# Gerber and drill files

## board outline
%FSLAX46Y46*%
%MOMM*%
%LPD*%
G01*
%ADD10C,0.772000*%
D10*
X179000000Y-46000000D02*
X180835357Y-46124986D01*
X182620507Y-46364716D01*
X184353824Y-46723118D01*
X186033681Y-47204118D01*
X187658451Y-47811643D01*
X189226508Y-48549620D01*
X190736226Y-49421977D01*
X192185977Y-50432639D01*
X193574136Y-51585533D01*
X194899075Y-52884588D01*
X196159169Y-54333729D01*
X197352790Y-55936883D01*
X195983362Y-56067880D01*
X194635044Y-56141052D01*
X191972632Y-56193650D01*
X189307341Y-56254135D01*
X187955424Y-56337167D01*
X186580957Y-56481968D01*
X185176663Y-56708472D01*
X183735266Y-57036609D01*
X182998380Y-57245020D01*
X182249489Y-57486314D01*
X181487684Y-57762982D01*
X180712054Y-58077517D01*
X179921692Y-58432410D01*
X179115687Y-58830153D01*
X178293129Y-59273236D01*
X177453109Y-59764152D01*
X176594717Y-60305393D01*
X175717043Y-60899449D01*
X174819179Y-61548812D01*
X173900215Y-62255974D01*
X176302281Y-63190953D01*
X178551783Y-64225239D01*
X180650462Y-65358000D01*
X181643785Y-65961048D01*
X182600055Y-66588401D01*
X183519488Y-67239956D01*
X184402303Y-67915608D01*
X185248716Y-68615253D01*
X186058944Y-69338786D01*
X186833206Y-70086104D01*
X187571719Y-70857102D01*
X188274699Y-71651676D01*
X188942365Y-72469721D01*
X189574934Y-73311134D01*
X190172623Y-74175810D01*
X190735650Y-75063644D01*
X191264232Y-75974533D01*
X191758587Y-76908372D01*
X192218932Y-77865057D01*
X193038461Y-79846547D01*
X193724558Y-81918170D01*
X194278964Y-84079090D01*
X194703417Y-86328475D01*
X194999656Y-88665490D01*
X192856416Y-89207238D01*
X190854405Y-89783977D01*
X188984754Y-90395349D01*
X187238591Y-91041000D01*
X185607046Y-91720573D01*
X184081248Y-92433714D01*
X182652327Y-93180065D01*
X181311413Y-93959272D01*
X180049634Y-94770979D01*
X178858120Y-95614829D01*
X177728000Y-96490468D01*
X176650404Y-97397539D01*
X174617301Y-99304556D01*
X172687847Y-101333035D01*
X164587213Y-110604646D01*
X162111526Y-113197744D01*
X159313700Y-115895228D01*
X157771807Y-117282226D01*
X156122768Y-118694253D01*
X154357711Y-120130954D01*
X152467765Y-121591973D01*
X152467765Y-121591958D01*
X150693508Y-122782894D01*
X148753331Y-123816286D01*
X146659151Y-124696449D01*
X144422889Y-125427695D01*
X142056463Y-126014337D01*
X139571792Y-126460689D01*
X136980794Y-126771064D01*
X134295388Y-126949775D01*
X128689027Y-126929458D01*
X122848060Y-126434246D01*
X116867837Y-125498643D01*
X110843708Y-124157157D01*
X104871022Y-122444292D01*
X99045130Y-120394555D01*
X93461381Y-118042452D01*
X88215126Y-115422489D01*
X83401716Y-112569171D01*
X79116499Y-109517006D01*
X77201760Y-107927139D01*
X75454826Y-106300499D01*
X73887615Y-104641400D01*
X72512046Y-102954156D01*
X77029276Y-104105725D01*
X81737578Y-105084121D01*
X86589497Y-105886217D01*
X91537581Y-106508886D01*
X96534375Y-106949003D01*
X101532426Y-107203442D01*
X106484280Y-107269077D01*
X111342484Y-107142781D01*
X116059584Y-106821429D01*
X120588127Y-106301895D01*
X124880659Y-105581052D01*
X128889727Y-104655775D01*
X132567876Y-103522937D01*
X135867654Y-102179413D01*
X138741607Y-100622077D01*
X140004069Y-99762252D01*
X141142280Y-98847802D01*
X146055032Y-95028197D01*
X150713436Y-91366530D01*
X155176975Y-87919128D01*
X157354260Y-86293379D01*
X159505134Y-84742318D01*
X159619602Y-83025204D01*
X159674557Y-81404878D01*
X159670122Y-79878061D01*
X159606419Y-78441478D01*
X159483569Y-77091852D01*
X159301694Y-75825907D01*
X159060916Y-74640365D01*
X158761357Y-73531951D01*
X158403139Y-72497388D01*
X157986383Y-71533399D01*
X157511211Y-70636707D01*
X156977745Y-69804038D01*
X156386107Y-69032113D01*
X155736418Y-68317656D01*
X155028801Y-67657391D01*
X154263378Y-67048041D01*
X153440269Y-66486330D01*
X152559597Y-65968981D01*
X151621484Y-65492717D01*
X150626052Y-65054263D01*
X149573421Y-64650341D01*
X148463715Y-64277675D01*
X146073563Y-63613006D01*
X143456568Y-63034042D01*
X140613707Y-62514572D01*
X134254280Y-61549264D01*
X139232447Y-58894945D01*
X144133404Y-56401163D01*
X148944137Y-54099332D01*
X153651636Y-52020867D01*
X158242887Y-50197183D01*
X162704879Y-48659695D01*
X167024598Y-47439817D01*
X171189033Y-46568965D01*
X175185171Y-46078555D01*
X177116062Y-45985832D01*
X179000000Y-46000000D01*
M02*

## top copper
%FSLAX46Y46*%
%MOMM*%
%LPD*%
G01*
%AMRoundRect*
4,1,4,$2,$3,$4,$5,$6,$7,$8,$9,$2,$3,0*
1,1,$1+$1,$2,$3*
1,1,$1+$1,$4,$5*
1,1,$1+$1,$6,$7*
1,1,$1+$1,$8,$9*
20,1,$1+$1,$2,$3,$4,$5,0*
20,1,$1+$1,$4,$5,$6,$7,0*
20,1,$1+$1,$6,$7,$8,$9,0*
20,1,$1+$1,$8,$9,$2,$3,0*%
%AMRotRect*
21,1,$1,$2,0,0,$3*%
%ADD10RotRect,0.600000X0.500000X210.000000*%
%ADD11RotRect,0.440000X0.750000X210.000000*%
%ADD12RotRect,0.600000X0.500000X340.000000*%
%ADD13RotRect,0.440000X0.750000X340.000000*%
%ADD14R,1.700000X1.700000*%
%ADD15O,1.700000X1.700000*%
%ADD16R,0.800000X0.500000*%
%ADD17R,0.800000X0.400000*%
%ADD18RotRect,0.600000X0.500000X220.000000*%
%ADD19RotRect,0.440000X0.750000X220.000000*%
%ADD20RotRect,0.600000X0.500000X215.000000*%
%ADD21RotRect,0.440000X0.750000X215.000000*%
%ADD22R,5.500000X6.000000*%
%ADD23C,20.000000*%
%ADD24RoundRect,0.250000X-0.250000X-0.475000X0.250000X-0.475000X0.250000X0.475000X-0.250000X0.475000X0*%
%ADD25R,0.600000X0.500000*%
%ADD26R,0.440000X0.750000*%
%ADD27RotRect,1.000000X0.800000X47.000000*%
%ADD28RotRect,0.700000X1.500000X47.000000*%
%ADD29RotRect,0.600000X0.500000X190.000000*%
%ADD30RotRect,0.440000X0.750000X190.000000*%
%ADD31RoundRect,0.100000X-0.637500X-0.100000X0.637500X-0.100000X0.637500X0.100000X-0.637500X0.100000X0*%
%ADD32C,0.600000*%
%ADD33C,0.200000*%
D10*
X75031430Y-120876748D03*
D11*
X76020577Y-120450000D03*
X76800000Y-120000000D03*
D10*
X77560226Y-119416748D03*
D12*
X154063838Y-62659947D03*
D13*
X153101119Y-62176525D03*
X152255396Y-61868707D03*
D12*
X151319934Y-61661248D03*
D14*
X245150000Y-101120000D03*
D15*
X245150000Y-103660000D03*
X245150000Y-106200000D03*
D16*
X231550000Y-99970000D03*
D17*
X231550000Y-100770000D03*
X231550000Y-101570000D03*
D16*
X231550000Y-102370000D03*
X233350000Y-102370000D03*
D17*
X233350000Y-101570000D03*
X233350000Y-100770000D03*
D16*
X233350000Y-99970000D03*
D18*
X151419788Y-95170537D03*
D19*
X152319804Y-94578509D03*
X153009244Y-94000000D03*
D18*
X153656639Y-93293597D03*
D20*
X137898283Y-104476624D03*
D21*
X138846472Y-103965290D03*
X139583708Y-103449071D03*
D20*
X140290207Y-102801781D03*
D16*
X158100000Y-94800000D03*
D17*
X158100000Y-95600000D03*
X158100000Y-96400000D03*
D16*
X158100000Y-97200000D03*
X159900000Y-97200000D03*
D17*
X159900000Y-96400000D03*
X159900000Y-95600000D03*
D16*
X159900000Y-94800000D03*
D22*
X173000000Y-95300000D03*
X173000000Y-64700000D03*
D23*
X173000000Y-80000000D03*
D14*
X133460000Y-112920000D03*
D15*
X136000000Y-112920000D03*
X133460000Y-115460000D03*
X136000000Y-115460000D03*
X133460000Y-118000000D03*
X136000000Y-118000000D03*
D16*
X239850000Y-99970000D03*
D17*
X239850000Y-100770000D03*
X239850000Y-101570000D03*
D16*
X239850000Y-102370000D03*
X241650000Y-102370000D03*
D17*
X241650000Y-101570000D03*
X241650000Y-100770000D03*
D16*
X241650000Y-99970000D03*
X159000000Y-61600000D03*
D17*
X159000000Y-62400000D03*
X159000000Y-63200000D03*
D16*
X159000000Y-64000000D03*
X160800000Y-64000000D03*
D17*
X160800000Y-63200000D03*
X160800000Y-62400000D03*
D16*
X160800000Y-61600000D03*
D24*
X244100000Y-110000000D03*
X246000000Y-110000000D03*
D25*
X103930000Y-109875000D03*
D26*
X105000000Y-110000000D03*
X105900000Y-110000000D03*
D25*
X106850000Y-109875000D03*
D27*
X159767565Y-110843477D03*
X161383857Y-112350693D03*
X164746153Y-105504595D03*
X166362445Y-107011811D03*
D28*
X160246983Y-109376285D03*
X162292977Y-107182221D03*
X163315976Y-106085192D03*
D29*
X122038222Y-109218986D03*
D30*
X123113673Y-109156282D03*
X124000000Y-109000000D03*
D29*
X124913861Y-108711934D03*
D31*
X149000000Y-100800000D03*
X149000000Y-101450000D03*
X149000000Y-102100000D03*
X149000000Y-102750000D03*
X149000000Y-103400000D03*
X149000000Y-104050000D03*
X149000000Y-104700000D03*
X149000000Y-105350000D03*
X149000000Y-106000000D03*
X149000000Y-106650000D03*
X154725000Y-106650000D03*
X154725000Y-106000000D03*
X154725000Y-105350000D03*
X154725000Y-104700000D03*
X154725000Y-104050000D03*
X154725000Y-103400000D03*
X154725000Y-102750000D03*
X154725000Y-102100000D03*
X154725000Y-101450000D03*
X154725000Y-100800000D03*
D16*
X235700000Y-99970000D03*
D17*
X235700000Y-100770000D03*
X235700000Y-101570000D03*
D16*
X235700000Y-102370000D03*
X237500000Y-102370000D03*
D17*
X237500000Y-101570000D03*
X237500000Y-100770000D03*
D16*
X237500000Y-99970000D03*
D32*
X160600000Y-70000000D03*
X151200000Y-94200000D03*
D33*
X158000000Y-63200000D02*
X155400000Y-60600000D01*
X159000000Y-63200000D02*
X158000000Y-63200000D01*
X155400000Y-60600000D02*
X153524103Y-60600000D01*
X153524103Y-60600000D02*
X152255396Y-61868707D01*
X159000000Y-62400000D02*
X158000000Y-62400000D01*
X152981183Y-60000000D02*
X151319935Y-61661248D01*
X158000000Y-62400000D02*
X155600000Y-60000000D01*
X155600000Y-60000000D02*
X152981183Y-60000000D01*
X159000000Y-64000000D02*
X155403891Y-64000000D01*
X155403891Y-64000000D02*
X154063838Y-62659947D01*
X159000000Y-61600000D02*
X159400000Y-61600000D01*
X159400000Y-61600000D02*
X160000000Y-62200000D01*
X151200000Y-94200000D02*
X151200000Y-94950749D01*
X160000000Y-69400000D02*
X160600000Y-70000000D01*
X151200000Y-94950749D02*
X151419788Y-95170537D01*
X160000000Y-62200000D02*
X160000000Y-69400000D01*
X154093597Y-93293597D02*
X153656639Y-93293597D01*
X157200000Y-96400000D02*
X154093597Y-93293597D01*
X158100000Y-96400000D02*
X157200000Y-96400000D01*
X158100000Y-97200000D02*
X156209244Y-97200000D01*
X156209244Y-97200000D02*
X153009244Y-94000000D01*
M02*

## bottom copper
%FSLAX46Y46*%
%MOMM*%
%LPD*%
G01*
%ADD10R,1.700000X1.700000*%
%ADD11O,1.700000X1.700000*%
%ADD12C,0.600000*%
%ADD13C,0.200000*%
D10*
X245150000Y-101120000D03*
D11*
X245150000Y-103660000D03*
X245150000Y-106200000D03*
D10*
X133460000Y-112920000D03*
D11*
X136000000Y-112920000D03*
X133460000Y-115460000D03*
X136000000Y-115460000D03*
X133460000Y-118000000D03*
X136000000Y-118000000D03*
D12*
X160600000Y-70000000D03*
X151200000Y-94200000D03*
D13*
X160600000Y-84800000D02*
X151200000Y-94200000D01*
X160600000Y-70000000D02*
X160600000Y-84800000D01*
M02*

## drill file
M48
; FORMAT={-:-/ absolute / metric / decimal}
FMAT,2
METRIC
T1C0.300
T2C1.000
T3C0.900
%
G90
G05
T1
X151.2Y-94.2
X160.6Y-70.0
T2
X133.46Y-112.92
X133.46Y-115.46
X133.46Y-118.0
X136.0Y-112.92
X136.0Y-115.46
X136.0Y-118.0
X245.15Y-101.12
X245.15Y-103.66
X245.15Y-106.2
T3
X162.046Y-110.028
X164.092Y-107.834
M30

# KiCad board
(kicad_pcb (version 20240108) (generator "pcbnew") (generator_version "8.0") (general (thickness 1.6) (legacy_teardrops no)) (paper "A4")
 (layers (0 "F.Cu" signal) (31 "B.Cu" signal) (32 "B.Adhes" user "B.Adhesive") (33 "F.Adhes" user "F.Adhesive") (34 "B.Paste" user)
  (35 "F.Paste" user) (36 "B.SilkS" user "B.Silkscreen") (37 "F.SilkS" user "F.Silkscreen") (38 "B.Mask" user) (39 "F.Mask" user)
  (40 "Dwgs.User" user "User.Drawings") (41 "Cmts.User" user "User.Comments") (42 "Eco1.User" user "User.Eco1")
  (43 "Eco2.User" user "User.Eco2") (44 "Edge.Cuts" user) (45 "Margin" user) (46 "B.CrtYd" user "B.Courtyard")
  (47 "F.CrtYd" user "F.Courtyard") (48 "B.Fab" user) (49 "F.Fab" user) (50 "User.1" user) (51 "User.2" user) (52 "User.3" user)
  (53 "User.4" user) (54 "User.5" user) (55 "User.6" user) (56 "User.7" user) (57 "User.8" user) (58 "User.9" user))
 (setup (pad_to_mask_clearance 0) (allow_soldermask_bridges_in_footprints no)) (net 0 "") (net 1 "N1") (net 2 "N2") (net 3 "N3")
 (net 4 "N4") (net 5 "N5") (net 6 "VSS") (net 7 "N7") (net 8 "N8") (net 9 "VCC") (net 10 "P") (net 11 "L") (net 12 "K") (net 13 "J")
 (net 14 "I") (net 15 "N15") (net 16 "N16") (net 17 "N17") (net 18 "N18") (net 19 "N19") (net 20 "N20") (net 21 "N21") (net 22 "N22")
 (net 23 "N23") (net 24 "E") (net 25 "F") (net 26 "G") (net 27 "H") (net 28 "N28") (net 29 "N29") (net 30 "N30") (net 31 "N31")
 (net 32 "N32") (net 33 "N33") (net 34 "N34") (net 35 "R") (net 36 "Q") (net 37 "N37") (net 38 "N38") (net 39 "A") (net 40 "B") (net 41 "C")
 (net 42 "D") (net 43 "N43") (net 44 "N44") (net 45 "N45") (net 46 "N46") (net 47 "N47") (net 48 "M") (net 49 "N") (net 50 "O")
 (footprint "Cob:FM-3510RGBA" (layer "F.Cu") (at 76.222789 119.900241 -150)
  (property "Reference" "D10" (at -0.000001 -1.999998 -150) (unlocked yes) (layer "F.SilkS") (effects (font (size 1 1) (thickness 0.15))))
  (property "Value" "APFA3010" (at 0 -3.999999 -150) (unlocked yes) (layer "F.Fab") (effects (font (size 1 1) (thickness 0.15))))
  (pad "1" smd rect (at 1.520001 -0.25 210) (size 0.6 0.5) (layers "F.Cu" "F.Paste" "F.Mask") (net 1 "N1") (thermal_bridge_angle 45))
  (pad "2" smd rect (at 0.45 -0.374999 210) (size 0.44 0.75) (layers "F.Cu" "F.Paste" "F.Mask") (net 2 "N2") (thermal_bridge_angle 45))
  (pad "3" smd rect (at -0.45 -0.374999 210) (size 0.44 0.75) (layers "F.Cu" "F.Paste" "F.Mask") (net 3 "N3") (thermal_bridge_angle 45))
  (pad "4" smd rect (at -1.400001 -0.250001 210) (size 0.6 0.5) (layers "F.Cu" "F.Paste" "F.Mask") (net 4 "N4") (thermal_bridge_angle 45)))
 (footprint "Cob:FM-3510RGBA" (layer "F.Cu") (at 152.55 62.375 -20)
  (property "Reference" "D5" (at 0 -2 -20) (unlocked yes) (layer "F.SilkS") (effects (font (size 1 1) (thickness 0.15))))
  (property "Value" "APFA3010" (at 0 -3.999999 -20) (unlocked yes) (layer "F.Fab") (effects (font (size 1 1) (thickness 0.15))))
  (pad "1" smd rect (at 1.52 -0.25 340) (size 0.6 0.5) (layers "F.Cu" "F.Paste" "F.Mask") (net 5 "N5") (thermal_bridge_angle 45))
  (pad "2" smd rect (at 0.45 -0.374999 340) (size 0.44 0.75) (layers "F.Cu" "F.Paste" "F.Mask") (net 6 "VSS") (thermal_bridge_angle 45))
  (pad "3" smd rect (at -0.45 -0.374999 340) (size 0.44 0.75) (layers "F.Cu" "F.Paste" "F.Mask") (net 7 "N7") (thermal_bridge_angle 45))
  (pad "4" smd rect (at -1.400001 -0.25 340) (size 0.6 0.5) (layers "F.Cu" "F.Paste" "F.Mask") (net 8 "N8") (thermal_bridge_angle 45)))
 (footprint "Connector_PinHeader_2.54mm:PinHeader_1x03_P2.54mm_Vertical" (layer "F.Cu") (at 245.15 101.12)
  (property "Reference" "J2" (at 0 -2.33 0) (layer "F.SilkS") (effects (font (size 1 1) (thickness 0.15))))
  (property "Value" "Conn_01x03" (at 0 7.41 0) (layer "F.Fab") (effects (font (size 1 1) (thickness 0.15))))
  (pad "1" thru_hole rect (at 0 0) (size 1.7 1.7) (drill 1) (layers "*.Cu" "*.Mask") (remove_unused_layers no) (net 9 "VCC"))
  (pad "2" thru_hole oval (at 0 2.54) (size 1.7 1.7) (drill 1) (layers "*.Cu" "*.Mask") (remove_unused_layers no) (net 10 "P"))
  (pad "3" thru_hole oval (at 0 5.08) (size 1.7 1.7) (drill 1) (layers "*.Cu" "*.Mask") (remove_unused_layers no) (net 6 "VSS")))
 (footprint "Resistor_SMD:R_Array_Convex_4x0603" (layer "F.Cu") (at 232.45 101.17)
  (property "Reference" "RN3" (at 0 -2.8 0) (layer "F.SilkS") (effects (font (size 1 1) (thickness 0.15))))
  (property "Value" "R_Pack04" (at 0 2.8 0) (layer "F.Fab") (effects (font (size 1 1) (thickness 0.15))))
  (pad "1" smd rect (at -0.9 -1.2) (size 0.8 0.5) (layers "F.Cu" "F.Paste" "F.Mask") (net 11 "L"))
  (pad "2" smd rect (at -0.9 -0.4) (size 0.8 0.4) (layers "F.Cu" "F.Paste" "F.Mask") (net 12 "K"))
  (pad "3" smd rect (at -0.9 0.4) (size 0.8 0.4) (layers "F.Cu" "F.Paste" "F.Mask") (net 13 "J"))
  (pad "4" smd rect (at -0.9 1.2) (size 0.8 0.5) (layers "F.Cu" "F.Paste" "F.Mask") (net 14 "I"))
  (pad "5" smd rect (at 0.9 1.2) (size 0.8 0.5) (layers "F.Cu" "F.Paste" "F.Mask") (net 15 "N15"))
  (pad "6" smd rect (at 0.9 0.4) (size 0.8 0.4) (layers "F.Cu" "F.Paste" "F.Mask") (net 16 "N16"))
  (pad "7" smd rect (at 0.9 -0.4) (size 0.8 0.4) (layers "F.Cu" "F.Paste" "F.Mask") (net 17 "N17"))
  (pad "8" smd rect (at 0.9 -1.2) (size 0.8 0.5) (layers "F.Cu" "F.Paste" "F.Mask") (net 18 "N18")))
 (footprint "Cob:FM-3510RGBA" (layer "F.Cu") (at 152.423479 94.001988 -140)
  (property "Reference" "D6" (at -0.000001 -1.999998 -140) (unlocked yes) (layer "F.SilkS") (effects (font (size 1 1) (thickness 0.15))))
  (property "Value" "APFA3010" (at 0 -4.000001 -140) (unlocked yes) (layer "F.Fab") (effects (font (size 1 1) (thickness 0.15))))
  (pad "1" smd rect (at 1.520001 -0.25 220) (size 0.6 0.5) (layers "F.Cu" "F.Paste" "F.Mask") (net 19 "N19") (thermal_bridge_angle 45))
  (pad "2" smd rect (at 0.45 -0.375 220) (size 0.44 0.75) (layers "F.Cu" "F.Paste" "F.Mask") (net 6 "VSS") (thermal_bridge_angle 45))
  (pad "3" smd rect (at -0.45 -0.375 220) (size 0.44 0.75) (layers "F.Cu" "F.Paste" "F.Mask") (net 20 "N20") (thermal_bridge_angle 45))
  (pad "4" smd rect (at -1.4 -0.250001 220) (size 0.6 0.5) (layers "F.Cu" "F.Paste" "F.Mask") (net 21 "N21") (thermal_bridge_angle 45)))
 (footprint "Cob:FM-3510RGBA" (layer "F.Cu") (at 139 103.4 -145)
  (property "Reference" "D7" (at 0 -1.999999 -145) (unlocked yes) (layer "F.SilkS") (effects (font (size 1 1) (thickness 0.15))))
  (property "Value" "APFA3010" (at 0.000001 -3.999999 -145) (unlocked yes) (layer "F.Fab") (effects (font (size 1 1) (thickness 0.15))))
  (pad "1" smd rect (at 1.52 -0.25 215) (size 0.6 0.5) (layers "F.Cu" "F.Paste" "F.Mask") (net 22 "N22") (thermal_bridge_angle 45))
  (pad "2" smd rect (at 0.45 -0.374998 215) (size 0.44 0.75) (layers "F.Cu" "F.Paste" "F.Mask") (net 6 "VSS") (thermal_bridge_angle 45))
  (pad "3" smd rect (at -0.45 -0.374998 215) (size 0.44 0.75) (layers "F.Cu" "F.Paste" "F.Mask") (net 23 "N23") (thermal_bridge_angle 45))
  (pad "4" smd rect (at -1.4 -0.25 215) (size 0.6 0.5) (layers "F.Cu" "F.Paste" "F.Mask") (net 15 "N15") (thermal_bridge_angle 45)))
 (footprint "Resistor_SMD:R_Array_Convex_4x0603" (layer "F.Cu") (at 159 96)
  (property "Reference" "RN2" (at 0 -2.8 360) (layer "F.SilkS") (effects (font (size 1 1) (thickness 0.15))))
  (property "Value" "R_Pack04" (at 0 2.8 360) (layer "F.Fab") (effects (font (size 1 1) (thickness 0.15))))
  (pad "1" smd rect (at -0.9 -1.2) (size 0.8 0.5) (layers "F.Cu" "F.Paste" "F.Mask") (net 23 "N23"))
  (pad "2" smd rect (at -0.9 -0.4) (size 0.8 0.4) (layers "F.Cu" "F.Paste" "F.Mask") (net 22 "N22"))
  (pad "3" smd rect (at -0.9 0.4) (size 0.8 0.4) (layers "F.Cu" "F.Paste" "F.Mask") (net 21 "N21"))
  (pad "4" smd rect (at -0.9 1.2) (size 0.8 0.5) (layers "F.Cu" "F.Paste" "F.Mask") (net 20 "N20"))
  (pad "5" smd rect (at 0.9 1.2) (size 0.8 0.5) (layers "F.Cu" "F.Paste" "F.Mask") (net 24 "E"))
  (pad "6" smd rect (at 0.9 0.4) (size 0.8 0.4) (layers "F.Cu" "F.Paste" "F.Mask") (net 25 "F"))
  (pad "7" smd rect (at 0.9 -0.4) (size 0.8 0.4) (layers "F.Cu" "F.Paste" "F.Mask") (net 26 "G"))
  (pad "8" smd rect (at 0.9 -1.2) (size 0.8 0.5) (layers "F.Cu" "F.Paste" "F.Mask") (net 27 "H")))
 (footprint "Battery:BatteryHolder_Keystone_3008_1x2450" (layer "F.Cu") (at 173 80 90)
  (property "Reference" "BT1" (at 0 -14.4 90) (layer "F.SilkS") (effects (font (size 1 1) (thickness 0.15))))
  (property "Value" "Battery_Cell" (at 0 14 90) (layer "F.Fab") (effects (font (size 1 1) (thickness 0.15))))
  (pad "1" smd rect (at -15.3 0 90) (size 6 5.5) (layers "F.Cu" "F.Paste" "F.Mask") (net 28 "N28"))
  (pad "1" smd rect (at 15.3 0 90) (size 6 5.5) (layers "F.Cu" "F.Paste" "F.Mask") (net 28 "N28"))
  (pad "2" smd circle (at 0 0 90) (size 20 20) (layers "F.Cu" "F.Mask") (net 6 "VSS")))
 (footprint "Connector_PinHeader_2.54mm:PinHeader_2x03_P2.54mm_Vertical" (layer "F.Cu") (at 133.46 112.92)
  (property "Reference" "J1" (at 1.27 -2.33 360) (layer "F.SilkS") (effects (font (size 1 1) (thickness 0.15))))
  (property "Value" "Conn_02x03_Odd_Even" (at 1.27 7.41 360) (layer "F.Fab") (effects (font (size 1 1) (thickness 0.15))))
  (pad "1" thru_hole rect (at 0 0) (size 1.7 1.7) (drill 1) (layers "*.Cu" "*.Mask") (remove_unused_layers no) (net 9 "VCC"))
  (pad "2" thru_hole oval (at 2.54 0) (size 1.7 1.7) (drill 1) (layers "*.Cu" "*.Mask") (remove_unused_layers no) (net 6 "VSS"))
  (pad "3" thru_hole oval (at 0 2.54) (size 1.7 1.7) (drill 1) (layers "*.Cu" "*.Mask") (remove_unused_layers no) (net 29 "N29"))
  (pad "4" thru_hole oval (at 2.54 2.54) (size 1.7 1.7) (drill 1) (layers "*.Cu" "*.Mask") (remove_unused_layers no) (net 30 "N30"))
  (pad "5" thru_hole oval (at 0 5.08) (size 1.7 1.7) (drill 1) (layers "*.Cu" "*.Mask") (remove_unused_layers no) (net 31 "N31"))
  (pad "6" thru_hole oval (at 2.54 5.08) (size 1.7 1.7) (drill 1) (layers "*.Cu" "*.Mask") (remove_unused_layers no) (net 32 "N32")))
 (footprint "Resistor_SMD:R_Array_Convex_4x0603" (layer "F.Cu") (at 240.75 101.17)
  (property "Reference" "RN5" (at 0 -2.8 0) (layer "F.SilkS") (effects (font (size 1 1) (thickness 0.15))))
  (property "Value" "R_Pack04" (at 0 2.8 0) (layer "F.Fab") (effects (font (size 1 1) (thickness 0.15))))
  (pad "1" smd rect (at -0.9 -1.2) (size 0.8 0.5) (layers "F.Cu" "F.Paste" "F.Mask") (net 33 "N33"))
  (pad "2" smd rect (at -0.9 -0.4) (size 0.8 0.4) (layers "F.Cu" "F.Paste" "F.Mask") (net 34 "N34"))
  (pad "3" smd rect (at -0.9 0.4) (size 0.8 0.4) (layers "F.Cu" "F.Paste" "F.Mask") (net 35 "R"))
  (pad "4" smd rect (at -0.9 1.2) (size 0.8 0.5) (layers "F.Cu" "F.Paste" "F.Mask") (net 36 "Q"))
  (pad "5" smd rect (at 0.9 1.2) (size 0.8 0.5) (layers "F.Cu" "F.Paste" "F.Mask") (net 3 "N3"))
  (pad "6" smd rect (at 0.9 0.4) (size 0.8 0.4) (layers "F.Cu" "F.Paste" "F.Mask") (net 4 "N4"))
  (pad "7" smd rect (at 0.9 -0.4) (size 0.8 0.4) (layers "F.Cu" "F.Paste" "F.Mask") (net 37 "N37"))
  (pad "8" smd rect (at 0.9 -1.2) (size 0.8 0.5) (layers "F.Cu" "F.Paste" "F.Mask") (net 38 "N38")))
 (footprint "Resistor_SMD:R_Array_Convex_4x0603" (layer "F.Cu") (at 159.9 62.8)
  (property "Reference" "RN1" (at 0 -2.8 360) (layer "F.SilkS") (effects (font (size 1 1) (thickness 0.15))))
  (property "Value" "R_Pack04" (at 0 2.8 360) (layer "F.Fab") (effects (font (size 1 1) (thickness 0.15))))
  (pad "1" smd rect (at -0.9 -1.2) (size 0.8 0.5) (layers "F.Cu" "F.Paste" "F.Mask") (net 19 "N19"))
  (pad "2" smd rect (at -0.9 -0.4) (size 0.8 0.4) (layers "F.Cu" "F.Paste" "F.Mask") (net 8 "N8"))
  (pad "3" smd rect (at -0.9 0.4) (size 0.8 0.4) (layers "F.Cu" "F.Paste" "F.Mask") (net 7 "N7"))
  (pad "4" smd rect (at -0.9 1.2) (size 0.8 0.5) (layers "F.Cu" "F.Paste" "F.Mask") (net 5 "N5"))
  (pad "5" smd rect (at 0.9 1.2) (size 0.8 0.5) (layers "F.Cu" "F.Paste" "F.Mask") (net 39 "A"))
  (pad "6" smd rect (at 0.9 0.4) (size 0.8 0.4) (layers "F.Cu" "F.Paste" "F.Mask") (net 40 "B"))
  (pad "7" smd rect (at 0.9 -0.4) (size 0.8 0.4) (layers "F.Cu" "F.Paste" "F.Mask") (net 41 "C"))
  (pad "8" smd rect (at 0.9 -1.2) (size 0.8 0.5) (layers "F.Cu" "F.Paste" "F.Mask") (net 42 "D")))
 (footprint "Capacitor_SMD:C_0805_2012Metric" (layer "F.Cu") (at 245.05 110)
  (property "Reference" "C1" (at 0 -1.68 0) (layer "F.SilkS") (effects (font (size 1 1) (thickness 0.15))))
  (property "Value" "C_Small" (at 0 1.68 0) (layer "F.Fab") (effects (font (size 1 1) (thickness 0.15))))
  (pad "1" smd roundrect (at -0.95 0) (size 1 1.45) (layers "F.Cu" "F.Paste" "F.Mask") (roundrect_rratio 0.25) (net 6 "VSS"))
  (pad "2" smd roundrect (at 0.95 0) (size 1 1.45) (layers "F.Cu" "F.Paste" "F.Mask") (roundrect_rratio 0.25) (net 9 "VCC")))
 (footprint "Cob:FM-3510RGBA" (layer "F.Cu") (at 105.45 109.625 180)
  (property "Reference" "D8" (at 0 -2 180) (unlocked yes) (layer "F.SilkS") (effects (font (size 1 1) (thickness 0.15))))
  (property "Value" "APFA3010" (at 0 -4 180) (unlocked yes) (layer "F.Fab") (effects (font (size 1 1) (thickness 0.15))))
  (pad "1" smd rect (at 1.52 -0.25 180) (size 0.6 0.5) (layers "F.Cu" "F.Paste" "F.Mask") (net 16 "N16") (thermal_bridge_angle 45))
  (pad "2" smd rect (at 0.45 -0.375 180) (size 0.44 0.75) (layers "F.Cu" "F.Paste" "F.Mask") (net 6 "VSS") (thermal_bridge_angle 45))
  (pad "3" smd rect (at -0.45 -0.375 180) (size 0.44 0.75) (layers "F.Cu" "F.Paste" "F.Mask") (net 17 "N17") (thermal_bridge_angle 45))
  (pad "4" smd rect (at -1.4 -0.25 180) (size 0.6 0.5) (layers "F.Cu" "F.Paste" "F.Mask") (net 18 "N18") (thermal_bridge_angle 45)))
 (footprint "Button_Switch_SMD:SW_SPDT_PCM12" (layer "F.Cu") (at 162.827315 108.705995 47)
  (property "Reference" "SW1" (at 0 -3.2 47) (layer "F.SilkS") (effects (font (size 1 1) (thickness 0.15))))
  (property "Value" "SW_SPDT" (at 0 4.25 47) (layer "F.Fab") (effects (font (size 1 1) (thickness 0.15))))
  (pad "" smd rect (at -3.65 -0.78 47) (size 1 0.8) (layers "F.Cu" "F.Paste" "F.Mask"))
  (pad "" smd rect (at -3.649999 1.43 47) (size 1 0.8) (layers "F.Cu" "F.Paste" "F.Mask"))
  (pad "" np_thru_hole circle (at -1.499999 0.330001 47) (size 0.9 0.9) (drill 0.9) (layers "*.Cu" "*.Mask"))
  (pad "" np_thru_hole circle (at 1.5 0.33 47) (size 0.9 0.9) (drill 0.9) (layers "*.Cu" "*.Mask"))
  (pad "" smd rect (at 3.65 -0.78 47) (size 1 0.8) (layers "F.Cu" "F.Paste" "F.Mask"))
  (pad "" smd rect (at 3.650001 1.43 47) (size 1 0.8) (layers "F.Cu" "F.Paste" "F.Mask"))
  (pad "1" smd rect (at -2.250001 -1.429999 47) (size 0.7 1.5) (layers "F.Cu" "F.Paste" "F.Mask") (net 9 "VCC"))
  (pad "2" smd rect (at 0.75 -1.430001 47) (size 0.7 1.5) (layers "F.Cu" "F.Paste" "F.Mask") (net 28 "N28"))
  (pad "3" smd rect (at 2.25 -1.429999 47) (size 0.7 1.5) (layers "F.Cu" "F.Paste" "F.Mask") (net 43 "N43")))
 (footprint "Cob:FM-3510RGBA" (layer "F.Cu") (at 123.491718 108.708839 -170)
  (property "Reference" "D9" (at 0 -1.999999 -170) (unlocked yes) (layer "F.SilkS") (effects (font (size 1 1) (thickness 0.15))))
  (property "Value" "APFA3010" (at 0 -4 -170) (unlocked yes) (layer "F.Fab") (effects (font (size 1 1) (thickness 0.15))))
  (pad "1" smd rect (at 1.52 -0.25 190) (size 0.6 0.5) (layers "F.Cu" "F.Paste" "F.Mask") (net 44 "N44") (thermal_bridge_angle 45))
  (pad "2" smd rect (at 0.449999 -0.374999 190) (size 0.44 0.75) (layers "F.Cu" "F.Paste" "F.Mask") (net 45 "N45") (thermal_bridge_angle 45))
  (pad "3" smd rect (at -0.45 -0.375 190) (size 0.44 0.75) (layers "F.Cu" "F.Paste" "F.Mask") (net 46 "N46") (thermal_bridge_angle 45))
  (pad "4" smd rect (at -1.4 -0.250001 190) (size 0.6 0.5) (layers "F.Cu" "F.Paste" "F.Mask") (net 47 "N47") (thermal_bridge_angle 45)))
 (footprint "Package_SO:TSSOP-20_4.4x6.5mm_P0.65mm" (layer "F.Cu") (at 151.8625 103.725)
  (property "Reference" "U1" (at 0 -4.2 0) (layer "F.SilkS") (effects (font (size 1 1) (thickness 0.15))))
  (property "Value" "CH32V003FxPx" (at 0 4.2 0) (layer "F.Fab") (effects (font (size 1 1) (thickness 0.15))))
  (pad "1" smd roundrect (at -2.8625 -2.925) (size 1.475 0.4) (layers "F.Cu" "F.Paste" "F.Mask") (roundrect_rratio 0.25) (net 39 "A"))
  (pad "2" smd roundrect (at -2.8625 -2.275) (size 1.475 0.4) (layers "F.Cu" "F.Paste" "F.Mask") (roundrect_rratio 0.25) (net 40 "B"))
  (pad "3" smd roundrect (at -2.8625 -1.625) (size 1.475 0.4) (layers "F.Cu" "F.Paste" "F.Mask") (roundrect_rratio 0.25) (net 41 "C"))
  (pad "4" smd roundrect (at -2.8625 -0.975) (size 1.475 0.4) (layers "F.Cu" "F.Paste" "F.Mask") (roundrect_rratio 0.25) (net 42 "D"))
  (pad "5" smd roundrect (at -2.8625 -0.325) (size 1.475 0.4) (layers "F.Cu" "F.Paste" "F.Mask") (roundrect_rratio 0.25) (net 24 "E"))
  (pad "6" smd roundrect (at -2.8625 0.325) (size 1.475 0.4) (layers "F.Cu" "F.Paste" "F.Mask") (roundrect_rratio 0.25) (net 25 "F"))
  (pad "7" smd roundrect (at -2.8625 0.975) (size 1.475 0.4) (layers "F.Cu" "F.Paste" "F.Mask") (roundrect_rratio 0.25) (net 6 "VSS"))
  (pad "8" smd roundrect (at -2.8625 1.625) (size 1.475 0.4) (layers "F.Cu" "F.Paste" "F.Mask") (roundrect_rratio 0.25) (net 26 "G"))
  (pad "9" smd roundrect (at -2.8625 2.275) (size 1.475 0.4) (layers "F.Cu" "F.Paste" "F.Mask") (roundrect_rratio 0.25) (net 9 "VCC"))
  (pad "10" smd roundrect (at -2.8625 2.925) (size 1.475 0.4) (layers "F.Cu" "F.Paste" "F.Mask") (roundrect_rratio 0.25) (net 27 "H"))
  (pad "11" smd roundrect (at 2.8625 2.925) (size 1.475 0.4) (layers "F.Cu" "F.Paste" "F.Mask") (roundrect_rratio 0.25) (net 14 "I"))
  (pad "12" smd roundrect (at 2.8625 2.275) (size 1.475 0.4) (layers "F.Cu" "F.Paste" "F.Mask") (roundrect_rratio 0.25) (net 13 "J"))
  (pad "13" smd roundrect (at 2.8625 1.625) (size 1.475 0.4) (layers "F.Cu" "F.Paste" "F.Mask") (roundrect_rratio 0.25) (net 12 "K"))
  (pad "14" smd roundrect (at 2.8625 0.975) (size 1.475 0.4) (layers "F.Cu" "F.Paste" "F.Mask") (roundrect_rratio 0.25) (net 11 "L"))
  (pad "15" smd roundrect (at 2.8625 0.325) (size 1.475 0.4) (layers "F.Cu" "F.Paste" "F.Mask") (roundrect_rratio 0.25) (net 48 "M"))
  (pad "16" smd roundrect (at 2.8625 -0.325) (size 1.475 0.4) (layers "F.Cu" "F.Paste" "F.Mask") (roundrect_rratio 0.25) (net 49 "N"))
  (pad "17" smd roundrect (at 2.8625 -0.975) (size 1.475 0.4) (layers "F.Cu" "F.Paste" "F.Mask") (roundrect_rratio 0.25) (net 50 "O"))
  (pad "18" smd roundrect (at 2.8625 -1.625) (size 1.475 0.4) (layers "F.Cu" "F.Paste" "F.Mask") (roundrect_rratio 0.25) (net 10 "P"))
  (pad "19" smd roundrect (at 2.8625 -2.275) (size 1.475 0.4) (layers "F.Cu" "F.Paste" "F.Mask") (roundrect_rratio 0.25) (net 36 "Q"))
  (pad "20" smd roundrect (at 2.8625 -2.925) (size 1.475 0.4) (layers "F.Cu" "F.Paste" "F.Mask") (roundrect_rratio 0.25) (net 35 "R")))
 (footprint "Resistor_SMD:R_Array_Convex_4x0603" (layer "F.Cu") (at 236.6 101.17)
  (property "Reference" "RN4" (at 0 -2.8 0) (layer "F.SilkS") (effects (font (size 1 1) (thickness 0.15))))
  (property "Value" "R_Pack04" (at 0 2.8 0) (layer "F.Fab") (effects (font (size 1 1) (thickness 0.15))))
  (pad "1" smd rect (at -0.9 -1.2) (size 0.8 0.5) (layers "F.Cu" "F.Paste" "F.Mask") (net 10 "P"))
  (pad "2" smd rect (at -0.9 -0.4) (size 0.8 0.4) (layers "F.Cu" "F.Paste" "F.Mask") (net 50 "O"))
  (pad "3" smd rect (at -0.9 0.4) (size 0.8 0.4) (layers "F.Cu" "F.Paste" "F.Mask") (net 49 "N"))
  (pad "4" smd rect (at -0.9 1.2) (size 0.8 0.5) (layers "F.Cu" "F.Paste" "F.Mask") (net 48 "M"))
  (pad "5" smd rect (at 0.9 1.2) (size 0.8 0.5) (layers "F.Cu" "F.Paste" "F.Mask") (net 44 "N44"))
  (pad "6" smd rect (at 0.9 0.4) (size 0.8 0.4) (layers "F.Cu" "F.Paste" "F.Mask") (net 46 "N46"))
  (pad "7" smd rect (at 0.9 -0.4) (size 0.8 0.4) (layers "F.Cu" "F.Paste" "F.Mask") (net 47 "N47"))
  (pad "8" smd rect (at 0.9 -1.2) (size 0.8 0.5) (layers "F.Cu" "F.Paste" "F.Mask") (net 1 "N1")))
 (gr_poly
  (pts (xy 179 46) (xy 180.835357 46.124986) (xy 182.620507 46.364716) (xy 184.353824 46.723118) (xy 186.033681 47.204118)
   (xy 187.658451 47.811643) (xy 189.226508 48.54962) (xy 190.736226 49.421977) (xy 192.185977 50.432639) (xy 193.574136 51.585533)
   (xy 194.899075 52.884588) (xy 196.159169 54.333729) (xy 197.35279 55.936883) (xy 195.983362 56.06788) (xy 194.635044 56.141052)
   (xy 191.972632 56.19365) (xy 189.307341 56.254135) (xy 187.955424 56.337167) (xy 186.580957 56.481968) (xy 185.176663 56.708472)
   (xy 183.735266 57.036609) (xy 182.99838 57.24502) (xy 182.249489 57.486314) (xy 181.487684 57.762982) (xy 180.712054 58.077517)
   (xy 179.921692 58.43241) (xy 179.115687 58.830153) (xy 178.293129 59.273236) (xy 177.453109 59.764152) (xy 176.594717 60.305393)
   (xy 175.717043 60.899449) (xy 174.819179 61.548812) (xy 173.900215 62.255974) (xy 176.302281 63.190953) (xy 178.551783 64.225239)
   (xy 180.650462 65.358) (xy 181.643785 65.961048) (xy 182.600055 66.588401) (xy 183.519488 67.239956) (xy 184.402303 67.915608)
   (xy 185.248716 68.615253) (xy 186.058944 69.338786) (xy 186.833206 70.086104) (xy 187.571719 70.857102) (xy 188.274699 71.651676)
   (xy 188.942365 72.469721) (xy 189.574934 73.311134) (xy 190.172623 74.17581) (xy 190.73565 75.063644) (xy 191.264232 75.974533)
   (xy 191.758587 76.908372) (xy 192.218932 77.865057) (xy 193.038461 79.846547) (xy 193.724558 81.91817) (xy 194.278964 84.07909)
   (xy 194.703417 86.328475) (xy 194.999656 88.66549) (xy 192.856416 89.207238) (xy 190.854405 89.783977) (xy 188.984754 90.395349)
   (xy 187.238591 91.041) (xy 185.607046 91.720573) (xy 184.081248 92.433714) (xy 182.652327 93.180065) (xy 181.311413 93.959272)
   (xy 180.049634 94.770979) (xy 178.85812 95.614829) (xy 177.728 96.490468) (xy 176.650404 97.397539) (xy 174.617301 99.304556)
   (xy 172.687847 101.333035) (xy 164.587213 110.604646) (xy 162.111526 113.197744) (xy 159.3137 115.895228) (xy 157.771807 117.282226)
   (xy 156.122768 118.694253) (xy 154.357711 120.130954) (xy 152.467765 121.591973) (xy 152.467765 121.591958) (xy 150.693508 122.782894)
   (xy 148.753331 123.816286) (xy 146.659151 124.696449) (xy 144.422889 125.427695) (xy 142.056463 126.014337) (xy 139.571792 126.460689)
   (xy 136.980794 126.771064) (xy 134.295388 126.949775) (xy 128.689027 126.929458) (xy 122.84806 126.434246) (xy 116.867837 125.498643)
   (xy 110.843708 124.157157) (xy 104.871022 122.444292) (xy 99.04513 120.394555) (xy 93.461381 118.042452) (xy 88.215126 115.422489)
   (xy 83.401716 112.569171) (xy 79.116499 109.517006) (xy 77.20176 107.927139) (xy 75.454826 106.300499) (xy 73.887615 104.6414)
   (xy 72.512046 102.954156) (xy 77.029276 104.105725) (xy 81.737578 105.084121) (xy 86.589497 105.886217) (xy 91.537581 106.508886)
   (xy 96.534375 106.949003) (xy 101.532426 107.203442) (xy 106.48428 107.269077) (xy 111.342484 107.142781) (xy 116.059584 106.821429)
   (xy 120.588127 106.301895) (xy 124.880659 105.581052) (xy 128.889727 104.655775) (xy 132.567876 103.522937) (xy 135.867654 102.179413)
   (xy 138.741607 100.622077) (xy 140.004069 99.762252) (xy 141.14228 98.847802) (xy 146.055032 95.028197) (xy 150.713436 91.36653)
   (xy 155.176975 87.919128) (xy 157.35426 86.293379) (xy 159.505134 84.742318) (xy 159.619602 83.025204) (xy 159.674557 81.404878)
   (xy 159.670122 79.878061) (xy 159.606419 78.441478) (xy 159.483569 77.091852) (xy 159.301694 75.825907) (xy 159.060916 74.640365)
   (xy 158.761357 73.531951) (xy 158.403139 72.497388) (xy 157.986383 71.533399) (xy 157.511211 70.636707) (xy 156.977745 69.804038)
   (xy 156.386107 69.032113) (xy 155.736418 68.317656) (xy 155.028801 67.657391) (xy 154.263378 67.048041) (xy 153.440269 66.48633)
   (xy 152.559597 65.968981) (xy 151.621484 65.492717) (xy 150.626052 65.054263) (xy 149.573421 64.650341) (xy 148.463715 64.277675)
   (xy 146.073563 63.613006) (xy 143.456568 63.034042) (xy 140.613707 62.514572) (xy 134.25428 61.549264) (xy 139.232447 58.894945)
   (xy 144.133404 56.401163) (xy 148.944137 54.099332) (xy 153.651636 52.020867) (xy 158.242887 50.197183) (xy 162.704879 48.659695)
   (xy 167.024598 47.439817) (xy 171.189033 46.568965) (xy 175.185171 46.078555) (xy 177.116062 45.985832))
  (stroke (width 0.772) (type solid) (color 255 0 0 1)) (fill none) (layer "Edge.Cuts"))
 (segment (start 158 63.2) (end 155.4 60.6) (width 0.2) (layer "F.Cu") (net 7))
 (segment (start 159 63.2) (end 158 63.2) (width 0.2) (layer "F.Cu") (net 7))
 (segment (start 155.4 60.6) (end 153.524103 60.6) (width 0.2) (layer "F.Cu") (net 7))
 (segment (start 153.524103 60.6) (end 152.255396 61.868707) (width 0.2) (layer "F.Cu") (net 7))
 (segment (start 159 62.4) (end 158 62.4) (width 0.2) (layer "F.Cu") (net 8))
 (segment (start 152.981183 60) (end 151.319935 61.661248) (width 0.2) (layer "F.Cu") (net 8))
 (segment (start 158 62.4) (end 155.6 60) (width 0.2) (layer "F.Cu") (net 8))
 (segment (start 155.6 60) (end 152.981183 60) (width 0.2) (layer "F.Cu") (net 8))
 (segment (start 159 64) (end 155.403891 64) (width 0.2) (layer "F.Cu") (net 5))
 (segment (start 155.403891 64) (end 154.063838 62.659947) (width 0.2) (layer "F.Cu") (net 5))
 (segment (start 159 61.6) (end 159.4 61.6) (width 0.2) (layer "F.Cu") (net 19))
 (segment (start 159.4 61.6) (end 160 62.2) (width 0.2) (layer "F.Cu") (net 19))
 (segment (start 151.2 94.2) (end 151.2 94.950749) (width 0.2) (layer "F.Cu") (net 19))
 (segment (start 160 69.4) (end 160.6 70) (width 0.2) (layer "F.Cu") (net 19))
 (segment (start 151.2 94.950749) (end 151.419788 95.170537) (width 0.2) (layer "F.Cu") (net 19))
 (segment (start 160 62.2) (end 160 69.4) (width 0.2) (layer "F.Cu") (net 19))
 (via (at 160.6 70) (size 0.6) (drill 0.3) (layers "F.Cu" "B.Cu") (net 19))
 (via (at 151.2 94.2) (size 0.6) (drill 0.3) (layers "F.Cu" "B.Cu") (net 19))
 (segment (start 160.6 84.8) (end 151.2 94.2) (width 0.2) (layer "B.Cu") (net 19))
 (segment (start 160.6 70) (end 160.6 84.8) (width 0.2) (layer "B.Cu") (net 19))
 (segment (start 154.093597 93.293597) (end 153.656639 93.293597) (width 0.2) (layer "F.Cu") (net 21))
 (segment (start 157.2 96.4) (end 154.093597 93.293597) (width 0.2) (layer "F.Cu") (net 21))
 (segment (start 158.1 96.4) (end 157.2 96.4) (width 0.2) (layer "F.Cu") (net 21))
 (segment (start 158.1 97.2) (end 156.209244 97.2) (width 0.2) (layer "F.Cu") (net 20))
 (segment (start 156.209244 97.2) (end 153.009244 94) (width 0.2) (layer "F.Cu") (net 20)))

